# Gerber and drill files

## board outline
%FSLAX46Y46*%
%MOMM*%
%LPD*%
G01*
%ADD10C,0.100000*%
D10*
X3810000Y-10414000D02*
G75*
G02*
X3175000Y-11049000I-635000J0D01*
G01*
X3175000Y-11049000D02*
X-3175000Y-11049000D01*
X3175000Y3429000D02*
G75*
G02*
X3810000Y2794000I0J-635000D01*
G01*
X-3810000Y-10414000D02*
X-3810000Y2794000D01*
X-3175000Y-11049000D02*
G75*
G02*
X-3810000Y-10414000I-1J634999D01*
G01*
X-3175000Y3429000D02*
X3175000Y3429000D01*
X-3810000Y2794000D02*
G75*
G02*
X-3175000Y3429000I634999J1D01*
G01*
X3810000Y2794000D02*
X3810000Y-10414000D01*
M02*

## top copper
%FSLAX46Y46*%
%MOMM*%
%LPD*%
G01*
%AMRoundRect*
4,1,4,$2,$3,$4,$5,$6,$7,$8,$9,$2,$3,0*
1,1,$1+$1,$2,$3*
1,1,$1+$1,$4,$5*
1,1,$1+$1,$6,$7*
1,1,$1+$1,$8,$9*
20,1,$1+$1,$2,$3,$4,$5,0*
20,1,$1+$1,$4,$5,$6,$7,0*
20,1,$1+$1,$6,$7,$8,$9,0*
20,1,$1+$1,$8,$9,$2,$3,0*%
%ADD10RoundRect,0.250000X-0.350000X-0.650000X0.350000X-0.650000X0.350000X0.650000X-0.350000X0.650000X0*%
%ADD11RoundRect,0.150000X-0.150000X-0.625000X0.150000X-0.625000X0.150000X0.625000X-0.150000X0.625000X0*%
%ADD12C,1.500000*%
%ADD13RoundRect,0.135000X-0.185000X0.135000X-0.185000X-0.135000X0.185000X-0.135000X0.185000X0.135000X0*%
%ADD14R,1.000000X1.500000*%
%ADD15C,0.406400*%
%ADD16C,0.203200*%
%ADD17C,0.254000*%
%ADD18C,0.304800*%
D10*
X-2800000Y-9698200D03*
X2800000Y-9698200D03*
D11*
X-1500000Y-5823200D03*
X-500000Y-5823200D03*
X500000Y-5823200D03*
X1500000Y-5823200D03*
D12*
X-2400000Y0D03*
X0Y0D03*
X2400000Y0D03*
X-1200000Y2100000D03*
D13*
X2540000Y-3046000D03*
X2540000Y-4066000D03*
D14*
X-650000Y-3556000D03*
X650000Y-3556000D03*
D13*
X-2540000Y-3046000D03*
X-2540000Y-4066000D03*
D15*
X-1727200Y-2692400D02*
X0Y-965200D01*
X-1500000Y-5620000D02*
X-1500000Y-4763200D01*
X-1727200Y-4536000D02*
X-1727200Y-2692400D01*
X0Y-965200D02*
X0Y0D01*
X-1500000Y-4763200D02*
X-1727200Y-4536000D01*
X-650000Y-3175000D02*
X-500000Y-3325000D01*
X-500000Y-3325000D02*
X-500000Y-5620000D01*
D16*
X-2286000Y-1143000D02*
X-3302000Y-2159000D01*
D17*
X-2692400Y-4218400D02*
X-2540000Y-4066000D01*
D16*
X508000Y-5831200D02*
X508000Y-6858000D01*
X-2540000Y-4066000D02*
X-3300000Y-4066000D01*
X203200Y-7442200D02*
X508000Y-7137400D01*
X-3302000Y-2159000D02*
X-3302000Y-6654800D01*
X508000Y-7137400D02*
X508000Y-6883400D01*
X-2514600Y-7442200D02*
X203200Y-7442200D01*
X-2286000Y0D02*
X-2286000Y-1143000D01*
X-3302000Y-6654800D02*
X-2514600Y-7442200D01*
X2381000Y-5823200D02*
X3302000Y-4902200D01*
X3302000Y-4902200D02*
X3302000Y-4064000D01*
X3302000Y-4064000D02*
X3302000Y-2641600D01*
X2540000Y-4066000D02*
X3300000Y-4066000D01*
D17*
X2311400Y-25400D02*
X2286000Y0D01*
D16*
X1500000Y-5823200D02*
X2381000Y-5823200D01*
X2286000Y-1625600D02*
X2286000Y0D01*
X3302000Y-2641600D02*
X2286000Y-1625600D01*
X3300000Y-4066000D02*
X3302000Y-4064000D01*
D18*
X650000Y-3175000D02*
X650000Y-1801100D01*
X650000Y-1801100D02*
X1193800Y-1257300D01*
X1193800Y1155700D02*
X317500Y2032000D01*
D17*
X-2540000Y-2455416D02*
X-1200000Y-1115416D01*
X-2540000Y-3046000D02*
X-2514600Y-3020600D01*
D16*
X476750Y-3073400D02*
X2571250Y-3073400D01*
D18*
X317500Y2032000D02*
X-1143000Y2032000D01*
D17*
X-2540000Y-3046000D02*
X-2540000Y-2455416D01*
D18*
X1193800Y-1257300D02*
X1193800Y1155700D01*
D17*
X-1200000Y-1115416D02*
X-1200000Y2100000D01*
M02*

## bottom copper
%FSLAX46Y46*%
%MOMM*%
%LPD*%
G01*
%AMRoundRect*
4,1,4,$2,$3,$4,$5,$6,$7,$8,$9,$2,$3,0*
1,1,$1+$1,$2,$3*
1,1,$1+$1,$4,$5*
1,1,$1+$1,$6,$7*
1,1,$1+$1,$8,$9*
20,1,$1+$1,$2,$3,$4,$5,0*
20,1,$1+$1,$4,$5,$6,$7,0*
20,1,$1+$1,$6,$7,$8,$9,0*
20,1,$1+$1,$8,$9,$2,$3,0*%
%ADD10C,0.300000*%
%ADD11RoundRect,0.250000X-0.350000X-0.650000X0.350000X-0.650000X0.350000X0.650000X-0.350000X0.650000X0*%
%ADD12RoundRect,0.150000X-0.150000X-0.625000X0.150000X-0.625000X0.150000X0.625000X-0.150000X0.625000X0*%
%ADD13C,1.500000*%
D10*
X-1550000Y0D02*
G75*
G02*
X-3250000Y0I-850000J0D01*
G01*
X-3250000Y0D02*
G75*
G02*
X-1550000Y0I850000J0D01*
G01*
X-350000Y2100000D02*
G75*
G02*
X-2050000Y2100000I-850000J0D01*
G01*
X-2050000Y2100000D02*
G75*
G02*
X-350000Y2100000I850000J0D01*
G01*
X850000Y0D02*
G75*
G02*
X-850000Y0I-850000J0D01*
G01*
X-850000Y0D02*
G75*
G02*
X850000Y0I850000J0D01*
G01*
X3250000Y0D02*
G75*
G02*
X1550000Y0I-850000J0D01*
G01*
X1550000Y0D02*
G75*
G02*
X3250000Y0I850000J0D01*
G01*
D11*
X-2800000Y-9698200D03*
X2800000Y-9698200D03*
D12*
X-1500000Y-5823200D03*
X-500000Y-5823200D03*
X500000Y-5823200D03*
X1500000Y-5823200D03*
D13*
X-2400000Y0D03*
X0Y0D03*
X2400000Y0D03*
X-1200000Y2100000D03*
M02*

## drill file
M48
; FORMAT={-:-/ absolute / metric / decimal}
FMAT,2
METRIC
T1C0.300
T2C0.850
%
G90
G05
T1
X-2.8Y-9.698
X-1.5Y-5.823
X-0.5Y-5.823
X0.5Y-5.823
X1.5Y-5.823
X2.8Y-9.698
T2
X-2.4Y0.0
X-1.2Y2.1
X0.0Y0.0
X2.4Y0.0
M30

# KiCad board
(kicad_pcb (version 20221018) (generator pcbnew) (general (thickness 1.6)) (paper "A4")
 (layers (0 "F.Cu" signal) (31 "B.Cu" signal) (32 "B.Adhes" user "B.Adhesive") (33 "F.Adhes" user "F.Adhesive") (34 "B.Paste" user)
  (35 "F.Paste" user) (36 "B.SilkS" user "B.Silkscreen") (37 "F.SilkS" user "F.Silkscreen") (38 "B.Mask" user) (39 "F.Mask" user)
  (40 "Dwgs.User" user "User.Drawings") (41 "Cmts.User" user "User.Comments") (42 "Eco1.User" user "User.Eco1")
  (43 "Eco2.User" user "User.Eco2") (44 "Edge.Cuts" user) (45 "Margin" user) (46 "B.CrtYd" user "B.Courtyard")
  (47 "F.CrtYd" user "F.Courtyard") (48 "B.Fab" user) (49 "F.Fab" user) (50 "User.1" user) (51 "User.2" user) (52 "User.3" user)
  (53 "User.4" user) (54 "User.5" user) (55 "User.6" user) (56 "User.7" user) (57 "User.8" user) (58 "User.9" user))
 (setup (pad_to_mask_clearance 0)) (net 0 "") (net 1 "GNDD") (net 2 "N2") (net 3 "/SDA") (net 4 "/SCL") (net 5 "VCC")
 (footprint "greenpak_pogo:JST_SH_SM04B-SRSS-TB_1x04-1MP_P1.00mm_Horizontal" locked (layer "F.Cu") (at 0 7.8232)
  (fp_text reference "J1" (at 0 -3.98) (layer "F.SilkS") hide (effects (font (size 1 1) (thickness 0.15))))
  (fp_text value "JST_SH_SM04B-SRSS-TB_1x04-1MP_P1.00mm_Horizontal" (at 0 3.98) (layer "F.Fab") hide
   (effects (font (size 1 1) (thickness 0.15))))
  (pad "" thru_hole roundrect locked (at -2.8 1.875) (size 1.2 1.8) (drill 0.3) (layers "*.Cu" "F.Paste" "F.Mask")
   (roundrect_rratio 0.2083333333))
  (pad "" thru_hole roundrect locked (at 2.8 1.875) (size 1.2 1.8) (drill 0.3) (layers "*.Cu" "F.Paste" "F.Mask")
   (roundrect_rratio 0.2083333333))
  (pad "1" thru_hole roundrect locked (at -1.5 -2) (size 0.6 1.55) (drill 0.3) (layers "*.Cu" "F.Paste" "F.Mask") (roundrect_rratio 0.25)
   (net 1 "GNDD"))
  (pad "2" thru_hole roundrect locked (at -0.5 -2) (size 0.6 1.55) (drill 0.3) (layers "*.Cu" "F.Paste" "F.Mask") (roundrect_rratio 0.25)
   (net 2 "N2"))
  (pad "3" thru_hole roundrect locked (at 0.5 -2) (size 0.6 1.55) (drill 0.3) (layers "*.Cu" "F.Paste" "F.Mask") (roundrect_rratio 0.25)
   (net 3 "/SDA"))
  (pad "4" thru_hole roundrect locked (at 1.5 -2) (size 0.6 1.55) (drill 0.3) (layers "*.Cu" "F.Paste" "F.Mask") (roundrect_rratio 0.25)
   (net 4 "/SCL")))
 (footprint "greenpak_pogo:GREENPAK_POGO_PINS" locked (layer "F.Cu") (at 0 0)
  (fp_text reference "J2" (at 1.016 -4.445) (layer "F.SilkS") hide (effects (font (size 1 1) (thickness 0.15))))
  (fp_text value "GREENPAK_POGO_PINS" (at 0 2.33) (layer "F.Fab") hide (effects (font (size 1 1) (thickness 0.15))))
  (fp_circle (center -2.4 0) (end -1.55 0) (stroke (width 0.3) (type solid)) (fill none) (layer "B.Cu"))
  (fp_circle (center -1.2 -2.1) (end -0.35 -2.1) (stroke (width 0.3) (type solid)) (fill none) (layer "B.Cu"))
  (fp_circle (center 0 0) (end 0.85 0) (stroke (width 0.3) (type solid)) (fill none) (layer "B.Cu"))
  (fp_circle (center 2.4 0) (end 3.25 0) (stroke (width 0.3) (type solid)) (fill none) (layer "B.Cu"))
  (pad "1" thru_hole circle locked (at -2.4 0) (size 1.5 1.5) (drill 0.85) (layers "*.Cu" "*.Mask") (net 3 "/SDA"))
  (pad "2" thru_hole circle locked (at 0 0) (size 1.5 1.5) (drill 0.85) (layers "*.Cu" "*.Mask") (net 1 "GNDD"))
  (pad "3" thru_hole circle locked (at 2.4 0) (size 1.5 1.5) (drill 0.85) (layers "*.Cu" "*.Mask") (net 4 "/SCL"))
  (pad "4" thru_hole circle locked (at -1.2 -2.1) (size 1.5 1.5) (drill 0.85) (layers "*.Cu" "*.Mask") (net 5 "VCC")))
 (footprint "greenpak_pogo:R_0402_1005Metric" (layer "F.Cu") (at 2.54 3.556 -90)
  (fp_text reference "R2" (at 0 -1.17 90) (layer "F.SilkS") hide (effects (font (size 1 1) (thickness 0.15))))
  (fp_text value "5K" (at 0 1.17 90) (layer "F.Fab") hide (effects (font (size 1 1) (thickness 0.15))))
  (pad "1" smd roundrect (at -0.51 0 270) (size 0.54 0.64) (layers "F.Cu" "F.Paste" "F.Mask") (roundrect_rratio 0.25) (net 5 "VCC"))
  (pad "2" smd roundrect (at 0.51 0 270) (size 0.54 0.64) (layers "F.Cu" "F.Paste" "F.Mask") (roundrect_rratio 0.25) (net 4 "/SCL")))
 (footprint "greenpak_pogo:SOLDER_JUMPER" (layer "F.Cu") (at 0 3.556)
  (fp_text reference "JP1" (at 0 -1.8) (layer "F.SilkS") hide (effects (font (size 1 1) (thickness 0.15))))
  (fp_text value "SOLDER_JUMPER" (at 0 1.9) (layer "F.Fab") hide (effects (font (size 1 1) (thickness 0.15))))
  (pad "1" smd rect (at -0.65 0) (size 1 1.5) (layers "F.Cu" "F.Mask") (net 2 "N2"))
  (pad "2" smd rect (at 0.65 0) (size 1 1.5) (layers "F.Cu" "F.Mask") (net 5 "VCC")))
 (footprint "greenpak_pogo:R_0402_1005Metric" (layer "F.Cu") (at -2.54 3.556 -90)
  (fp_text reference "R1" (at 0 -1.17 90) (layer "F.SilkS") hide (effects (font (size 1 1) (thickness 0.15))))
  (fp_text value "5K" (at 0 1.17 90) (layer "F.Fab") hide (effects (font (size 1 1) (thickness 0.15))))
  (pad "1" smd roundrect (at -0.51 0 270) (size 0.54 0.64) (layers "F.Cu" "F.Paste" "F.Mask") (roundrect_rratio 0.25) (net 5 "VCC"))
  (pad "2" smd roundrect (at 0.51 0 270) (size 0.54 0.64) (layers "F.Cu" "F.Paste" "F.Mask") (roundrect_rratio 0.25) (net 3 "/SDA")))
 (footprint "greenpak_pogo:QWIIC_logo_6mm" (layer "B.Cu") (at 0.040263 4.7302 180)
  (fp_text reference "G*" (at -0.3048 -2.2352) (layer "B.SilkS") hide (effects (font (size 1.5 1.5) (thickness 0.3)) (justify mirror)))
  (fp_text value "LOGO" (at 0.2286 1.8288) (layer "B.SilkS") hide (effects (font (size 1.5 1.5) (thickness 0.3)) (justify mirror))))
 (gr_arc (start 3.81 10.414) (mid 3.624013 10.863013) (end 3.175 11.049) (stroke (width 0.1) (type default)) (layer "Edge.Cuts"))
 (gr_line (start 3.175 11.049) (end -3.175 11.049) (stroke (width 0.1) (type default)) (layer "Edge.Cuts"))
 (gr_arc (start 3.175 -3.429) (mid 3.624013 -3.243013) (end 3.81 -2.794) (stroke (width 0.1) (type default)) (layer "Edge.Cuts"))
 (gr_line (start -3.81 10.414) (end -3.81 -2.794) (stroke (width 0.1) (type default)) (layer "Edge.Cuts"))
 (gr_arc (start -3.175 11.049) (mid -3.624013 10.863013) (end -3.81 10.414) (stroke (width 0.1) (type default)) (layer "Edge.Cuts"))
 (gr_line (start -3.175 -3.429) (end 3.175 -3.429) (stroke (width 0.1) (type default)) (layer "Edge.Cuts"))
 (gr_arc (start -3.81 -2.794) (mid -3.624013 -3.243013) (end -3.175 -3.429) (stroke (width 0.1) (type default)) (layer "Edge.Cuts"))
 (gr_line (start 3.81 -2.794) (end 3.81 10.414) (stroke (width 0.1) (type default)) (layer "Edge.Cuts"))
 (segment (start -1.7272 2.6924) (end 0 0.9652) (width 0.4064) (layer "F.Cu") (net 1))
 (segment (start -1.5 5.62) (end -1.5 4.7632) (width 0.4064) (layer "F.Cu") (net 1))
 (segment (start -1.7272 4.536) (end -1.7272 2.6924) (width 0.4064) (layer "F.Cu") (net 1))
 (segment (start 0 0.9652) (end 0 0) (width 0.4064) (layer "F.Cu") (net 1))
 (segment (start -1.5 4.7632) (end -1.7272 4.536) (width 0.4064) (layer "F.Cu") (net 1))
 (segment (start -0.65 3.175) (end -0.5 3.325) (width 0.4064) (layer "F.Cu") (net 2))
 (segment (start -0.5 3.325) (end -0.5 5.62) (width 0.4064) (layer "F.Cu") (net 2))
 (segment (start -2.286 1.143) (end -3.302 2.159) (width 0.2032) (layer "F.Cu") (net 3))
 (segment (start -2.6924 4.2184) (end -2.54 4.066) (width 0.254) (layer "F.Cu") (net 3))
 (segment (start 0.508 5.8312) (end 0.508 6.858) (width 0.2032) (layer "F.Cu") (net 3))
 (segment (start -2.54 4.066) (end -3.3 4.066) (width 0.2032) (layer "F.Cu") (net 3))
 (segment (start 0.2032 7.4422) (end 0.508 7.1374) (width 0.2032) (layer "F.Cu") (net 3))
 (segment (start -3.302 2.159) (end -3.302 6.6548) (width 0.2032) (layer "F.Cu") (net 3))
 (segment (start 0.508 7.1374) (end 0.508 6.8834) (width 0.2032) (layer "F.Cu") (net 3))
 (segment (start -2.5146 7.4422) (end 0.2032 7.4422) (width 0.2032) (layer "F.Cu") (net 3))
 (segment (start -2.286 0) (end -2.286 1.143) (width 0.2032) (layer "F.Cu") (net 3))
 (segment (start -3.302 6.6548) (end -2.5146 7.4422) (width 0.2032) (layer "F.Cu") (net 3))
 (segment (start 2.381 5.8232) (end 3.302 4.9022) (width 0.2032) (layer "F.Cu") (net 4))
 (segment (start 3.302 4.9022) (end 3.302 4.064) (width 0.2032) (layer "F.Cu") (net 4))
 (segment (start 3.302 4.064) (end 3.302 2.6416) (width 0.2032) (layer "F.Cu") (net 4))
 (segment (start 2.54 4.066) (end 3.3 4.066) (width 0.2032) (layer "F.Cu") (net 4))
 (segment (start 2.3114 0.0254) (end 2.286 0) (width 0.254) (layer "F.Cu") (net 4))
 (segment (start 1.5 5.8232) (end 2.381 5.8232) (width 0.2032) (layer "F.Cu") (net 4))
 (segment (start 2.286 1.6256) (end 2.286 0) (width 0.2032) (layer "F.Cu") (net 4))
 (segment (start 3.302 2.6416) (end 2.286 1.6256) (width 0.2032) (layer "F.Cu") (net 4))
 (segment (start 3.3 4.066) (end 3.302 4.064) (width 0.2032) (layer "F.Cu") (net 4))
 (segment (start 0.65 3.175) (end 0.65 1.8011) (width 0.3048) (layer "F.Cu") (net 5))
 (segment (start 0.65 1.8011) (end 1.1938 1.2573) (width 0.3048) (layer "F.Cu") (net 5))
 (segment (start 1.1938 -1.1557) (end 0.3175 -2.032) (width 0.3048) (layer "F.Cu") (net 5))
 (segment (start -2.54 2.455416) (end -1.2 1.115416) (width 0.254) (layer "F.Cu") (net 5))
 (segment (start -2.54 3.046) (end -2.5146 3.0206) (width 0.254) (layer "F.Cu") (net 5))
 (segment (start 0.47675 3.0734) (end 2.57125 3.0734) (width 0.2032) (layer "F.Cu") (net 5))
 (segment (start 0.3175 -2.032) (end -1.143 -2.032) (width 0.3048) (layer "F.Cu") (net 5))
 (segment (start -2.54 3.046) (end -2.54 2.455416) (width 0.254) (layer "F.Cu") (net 5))
 (segment (start 1.1938 1.2573) (end 1.1938 -1.1557) (width 0.3048) (layer "F.Cu") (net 5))
 (segment (start -1.2 1.115416) (end -1.2 -2.1) (width 0.254) (layer "F.Cu") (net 5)))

